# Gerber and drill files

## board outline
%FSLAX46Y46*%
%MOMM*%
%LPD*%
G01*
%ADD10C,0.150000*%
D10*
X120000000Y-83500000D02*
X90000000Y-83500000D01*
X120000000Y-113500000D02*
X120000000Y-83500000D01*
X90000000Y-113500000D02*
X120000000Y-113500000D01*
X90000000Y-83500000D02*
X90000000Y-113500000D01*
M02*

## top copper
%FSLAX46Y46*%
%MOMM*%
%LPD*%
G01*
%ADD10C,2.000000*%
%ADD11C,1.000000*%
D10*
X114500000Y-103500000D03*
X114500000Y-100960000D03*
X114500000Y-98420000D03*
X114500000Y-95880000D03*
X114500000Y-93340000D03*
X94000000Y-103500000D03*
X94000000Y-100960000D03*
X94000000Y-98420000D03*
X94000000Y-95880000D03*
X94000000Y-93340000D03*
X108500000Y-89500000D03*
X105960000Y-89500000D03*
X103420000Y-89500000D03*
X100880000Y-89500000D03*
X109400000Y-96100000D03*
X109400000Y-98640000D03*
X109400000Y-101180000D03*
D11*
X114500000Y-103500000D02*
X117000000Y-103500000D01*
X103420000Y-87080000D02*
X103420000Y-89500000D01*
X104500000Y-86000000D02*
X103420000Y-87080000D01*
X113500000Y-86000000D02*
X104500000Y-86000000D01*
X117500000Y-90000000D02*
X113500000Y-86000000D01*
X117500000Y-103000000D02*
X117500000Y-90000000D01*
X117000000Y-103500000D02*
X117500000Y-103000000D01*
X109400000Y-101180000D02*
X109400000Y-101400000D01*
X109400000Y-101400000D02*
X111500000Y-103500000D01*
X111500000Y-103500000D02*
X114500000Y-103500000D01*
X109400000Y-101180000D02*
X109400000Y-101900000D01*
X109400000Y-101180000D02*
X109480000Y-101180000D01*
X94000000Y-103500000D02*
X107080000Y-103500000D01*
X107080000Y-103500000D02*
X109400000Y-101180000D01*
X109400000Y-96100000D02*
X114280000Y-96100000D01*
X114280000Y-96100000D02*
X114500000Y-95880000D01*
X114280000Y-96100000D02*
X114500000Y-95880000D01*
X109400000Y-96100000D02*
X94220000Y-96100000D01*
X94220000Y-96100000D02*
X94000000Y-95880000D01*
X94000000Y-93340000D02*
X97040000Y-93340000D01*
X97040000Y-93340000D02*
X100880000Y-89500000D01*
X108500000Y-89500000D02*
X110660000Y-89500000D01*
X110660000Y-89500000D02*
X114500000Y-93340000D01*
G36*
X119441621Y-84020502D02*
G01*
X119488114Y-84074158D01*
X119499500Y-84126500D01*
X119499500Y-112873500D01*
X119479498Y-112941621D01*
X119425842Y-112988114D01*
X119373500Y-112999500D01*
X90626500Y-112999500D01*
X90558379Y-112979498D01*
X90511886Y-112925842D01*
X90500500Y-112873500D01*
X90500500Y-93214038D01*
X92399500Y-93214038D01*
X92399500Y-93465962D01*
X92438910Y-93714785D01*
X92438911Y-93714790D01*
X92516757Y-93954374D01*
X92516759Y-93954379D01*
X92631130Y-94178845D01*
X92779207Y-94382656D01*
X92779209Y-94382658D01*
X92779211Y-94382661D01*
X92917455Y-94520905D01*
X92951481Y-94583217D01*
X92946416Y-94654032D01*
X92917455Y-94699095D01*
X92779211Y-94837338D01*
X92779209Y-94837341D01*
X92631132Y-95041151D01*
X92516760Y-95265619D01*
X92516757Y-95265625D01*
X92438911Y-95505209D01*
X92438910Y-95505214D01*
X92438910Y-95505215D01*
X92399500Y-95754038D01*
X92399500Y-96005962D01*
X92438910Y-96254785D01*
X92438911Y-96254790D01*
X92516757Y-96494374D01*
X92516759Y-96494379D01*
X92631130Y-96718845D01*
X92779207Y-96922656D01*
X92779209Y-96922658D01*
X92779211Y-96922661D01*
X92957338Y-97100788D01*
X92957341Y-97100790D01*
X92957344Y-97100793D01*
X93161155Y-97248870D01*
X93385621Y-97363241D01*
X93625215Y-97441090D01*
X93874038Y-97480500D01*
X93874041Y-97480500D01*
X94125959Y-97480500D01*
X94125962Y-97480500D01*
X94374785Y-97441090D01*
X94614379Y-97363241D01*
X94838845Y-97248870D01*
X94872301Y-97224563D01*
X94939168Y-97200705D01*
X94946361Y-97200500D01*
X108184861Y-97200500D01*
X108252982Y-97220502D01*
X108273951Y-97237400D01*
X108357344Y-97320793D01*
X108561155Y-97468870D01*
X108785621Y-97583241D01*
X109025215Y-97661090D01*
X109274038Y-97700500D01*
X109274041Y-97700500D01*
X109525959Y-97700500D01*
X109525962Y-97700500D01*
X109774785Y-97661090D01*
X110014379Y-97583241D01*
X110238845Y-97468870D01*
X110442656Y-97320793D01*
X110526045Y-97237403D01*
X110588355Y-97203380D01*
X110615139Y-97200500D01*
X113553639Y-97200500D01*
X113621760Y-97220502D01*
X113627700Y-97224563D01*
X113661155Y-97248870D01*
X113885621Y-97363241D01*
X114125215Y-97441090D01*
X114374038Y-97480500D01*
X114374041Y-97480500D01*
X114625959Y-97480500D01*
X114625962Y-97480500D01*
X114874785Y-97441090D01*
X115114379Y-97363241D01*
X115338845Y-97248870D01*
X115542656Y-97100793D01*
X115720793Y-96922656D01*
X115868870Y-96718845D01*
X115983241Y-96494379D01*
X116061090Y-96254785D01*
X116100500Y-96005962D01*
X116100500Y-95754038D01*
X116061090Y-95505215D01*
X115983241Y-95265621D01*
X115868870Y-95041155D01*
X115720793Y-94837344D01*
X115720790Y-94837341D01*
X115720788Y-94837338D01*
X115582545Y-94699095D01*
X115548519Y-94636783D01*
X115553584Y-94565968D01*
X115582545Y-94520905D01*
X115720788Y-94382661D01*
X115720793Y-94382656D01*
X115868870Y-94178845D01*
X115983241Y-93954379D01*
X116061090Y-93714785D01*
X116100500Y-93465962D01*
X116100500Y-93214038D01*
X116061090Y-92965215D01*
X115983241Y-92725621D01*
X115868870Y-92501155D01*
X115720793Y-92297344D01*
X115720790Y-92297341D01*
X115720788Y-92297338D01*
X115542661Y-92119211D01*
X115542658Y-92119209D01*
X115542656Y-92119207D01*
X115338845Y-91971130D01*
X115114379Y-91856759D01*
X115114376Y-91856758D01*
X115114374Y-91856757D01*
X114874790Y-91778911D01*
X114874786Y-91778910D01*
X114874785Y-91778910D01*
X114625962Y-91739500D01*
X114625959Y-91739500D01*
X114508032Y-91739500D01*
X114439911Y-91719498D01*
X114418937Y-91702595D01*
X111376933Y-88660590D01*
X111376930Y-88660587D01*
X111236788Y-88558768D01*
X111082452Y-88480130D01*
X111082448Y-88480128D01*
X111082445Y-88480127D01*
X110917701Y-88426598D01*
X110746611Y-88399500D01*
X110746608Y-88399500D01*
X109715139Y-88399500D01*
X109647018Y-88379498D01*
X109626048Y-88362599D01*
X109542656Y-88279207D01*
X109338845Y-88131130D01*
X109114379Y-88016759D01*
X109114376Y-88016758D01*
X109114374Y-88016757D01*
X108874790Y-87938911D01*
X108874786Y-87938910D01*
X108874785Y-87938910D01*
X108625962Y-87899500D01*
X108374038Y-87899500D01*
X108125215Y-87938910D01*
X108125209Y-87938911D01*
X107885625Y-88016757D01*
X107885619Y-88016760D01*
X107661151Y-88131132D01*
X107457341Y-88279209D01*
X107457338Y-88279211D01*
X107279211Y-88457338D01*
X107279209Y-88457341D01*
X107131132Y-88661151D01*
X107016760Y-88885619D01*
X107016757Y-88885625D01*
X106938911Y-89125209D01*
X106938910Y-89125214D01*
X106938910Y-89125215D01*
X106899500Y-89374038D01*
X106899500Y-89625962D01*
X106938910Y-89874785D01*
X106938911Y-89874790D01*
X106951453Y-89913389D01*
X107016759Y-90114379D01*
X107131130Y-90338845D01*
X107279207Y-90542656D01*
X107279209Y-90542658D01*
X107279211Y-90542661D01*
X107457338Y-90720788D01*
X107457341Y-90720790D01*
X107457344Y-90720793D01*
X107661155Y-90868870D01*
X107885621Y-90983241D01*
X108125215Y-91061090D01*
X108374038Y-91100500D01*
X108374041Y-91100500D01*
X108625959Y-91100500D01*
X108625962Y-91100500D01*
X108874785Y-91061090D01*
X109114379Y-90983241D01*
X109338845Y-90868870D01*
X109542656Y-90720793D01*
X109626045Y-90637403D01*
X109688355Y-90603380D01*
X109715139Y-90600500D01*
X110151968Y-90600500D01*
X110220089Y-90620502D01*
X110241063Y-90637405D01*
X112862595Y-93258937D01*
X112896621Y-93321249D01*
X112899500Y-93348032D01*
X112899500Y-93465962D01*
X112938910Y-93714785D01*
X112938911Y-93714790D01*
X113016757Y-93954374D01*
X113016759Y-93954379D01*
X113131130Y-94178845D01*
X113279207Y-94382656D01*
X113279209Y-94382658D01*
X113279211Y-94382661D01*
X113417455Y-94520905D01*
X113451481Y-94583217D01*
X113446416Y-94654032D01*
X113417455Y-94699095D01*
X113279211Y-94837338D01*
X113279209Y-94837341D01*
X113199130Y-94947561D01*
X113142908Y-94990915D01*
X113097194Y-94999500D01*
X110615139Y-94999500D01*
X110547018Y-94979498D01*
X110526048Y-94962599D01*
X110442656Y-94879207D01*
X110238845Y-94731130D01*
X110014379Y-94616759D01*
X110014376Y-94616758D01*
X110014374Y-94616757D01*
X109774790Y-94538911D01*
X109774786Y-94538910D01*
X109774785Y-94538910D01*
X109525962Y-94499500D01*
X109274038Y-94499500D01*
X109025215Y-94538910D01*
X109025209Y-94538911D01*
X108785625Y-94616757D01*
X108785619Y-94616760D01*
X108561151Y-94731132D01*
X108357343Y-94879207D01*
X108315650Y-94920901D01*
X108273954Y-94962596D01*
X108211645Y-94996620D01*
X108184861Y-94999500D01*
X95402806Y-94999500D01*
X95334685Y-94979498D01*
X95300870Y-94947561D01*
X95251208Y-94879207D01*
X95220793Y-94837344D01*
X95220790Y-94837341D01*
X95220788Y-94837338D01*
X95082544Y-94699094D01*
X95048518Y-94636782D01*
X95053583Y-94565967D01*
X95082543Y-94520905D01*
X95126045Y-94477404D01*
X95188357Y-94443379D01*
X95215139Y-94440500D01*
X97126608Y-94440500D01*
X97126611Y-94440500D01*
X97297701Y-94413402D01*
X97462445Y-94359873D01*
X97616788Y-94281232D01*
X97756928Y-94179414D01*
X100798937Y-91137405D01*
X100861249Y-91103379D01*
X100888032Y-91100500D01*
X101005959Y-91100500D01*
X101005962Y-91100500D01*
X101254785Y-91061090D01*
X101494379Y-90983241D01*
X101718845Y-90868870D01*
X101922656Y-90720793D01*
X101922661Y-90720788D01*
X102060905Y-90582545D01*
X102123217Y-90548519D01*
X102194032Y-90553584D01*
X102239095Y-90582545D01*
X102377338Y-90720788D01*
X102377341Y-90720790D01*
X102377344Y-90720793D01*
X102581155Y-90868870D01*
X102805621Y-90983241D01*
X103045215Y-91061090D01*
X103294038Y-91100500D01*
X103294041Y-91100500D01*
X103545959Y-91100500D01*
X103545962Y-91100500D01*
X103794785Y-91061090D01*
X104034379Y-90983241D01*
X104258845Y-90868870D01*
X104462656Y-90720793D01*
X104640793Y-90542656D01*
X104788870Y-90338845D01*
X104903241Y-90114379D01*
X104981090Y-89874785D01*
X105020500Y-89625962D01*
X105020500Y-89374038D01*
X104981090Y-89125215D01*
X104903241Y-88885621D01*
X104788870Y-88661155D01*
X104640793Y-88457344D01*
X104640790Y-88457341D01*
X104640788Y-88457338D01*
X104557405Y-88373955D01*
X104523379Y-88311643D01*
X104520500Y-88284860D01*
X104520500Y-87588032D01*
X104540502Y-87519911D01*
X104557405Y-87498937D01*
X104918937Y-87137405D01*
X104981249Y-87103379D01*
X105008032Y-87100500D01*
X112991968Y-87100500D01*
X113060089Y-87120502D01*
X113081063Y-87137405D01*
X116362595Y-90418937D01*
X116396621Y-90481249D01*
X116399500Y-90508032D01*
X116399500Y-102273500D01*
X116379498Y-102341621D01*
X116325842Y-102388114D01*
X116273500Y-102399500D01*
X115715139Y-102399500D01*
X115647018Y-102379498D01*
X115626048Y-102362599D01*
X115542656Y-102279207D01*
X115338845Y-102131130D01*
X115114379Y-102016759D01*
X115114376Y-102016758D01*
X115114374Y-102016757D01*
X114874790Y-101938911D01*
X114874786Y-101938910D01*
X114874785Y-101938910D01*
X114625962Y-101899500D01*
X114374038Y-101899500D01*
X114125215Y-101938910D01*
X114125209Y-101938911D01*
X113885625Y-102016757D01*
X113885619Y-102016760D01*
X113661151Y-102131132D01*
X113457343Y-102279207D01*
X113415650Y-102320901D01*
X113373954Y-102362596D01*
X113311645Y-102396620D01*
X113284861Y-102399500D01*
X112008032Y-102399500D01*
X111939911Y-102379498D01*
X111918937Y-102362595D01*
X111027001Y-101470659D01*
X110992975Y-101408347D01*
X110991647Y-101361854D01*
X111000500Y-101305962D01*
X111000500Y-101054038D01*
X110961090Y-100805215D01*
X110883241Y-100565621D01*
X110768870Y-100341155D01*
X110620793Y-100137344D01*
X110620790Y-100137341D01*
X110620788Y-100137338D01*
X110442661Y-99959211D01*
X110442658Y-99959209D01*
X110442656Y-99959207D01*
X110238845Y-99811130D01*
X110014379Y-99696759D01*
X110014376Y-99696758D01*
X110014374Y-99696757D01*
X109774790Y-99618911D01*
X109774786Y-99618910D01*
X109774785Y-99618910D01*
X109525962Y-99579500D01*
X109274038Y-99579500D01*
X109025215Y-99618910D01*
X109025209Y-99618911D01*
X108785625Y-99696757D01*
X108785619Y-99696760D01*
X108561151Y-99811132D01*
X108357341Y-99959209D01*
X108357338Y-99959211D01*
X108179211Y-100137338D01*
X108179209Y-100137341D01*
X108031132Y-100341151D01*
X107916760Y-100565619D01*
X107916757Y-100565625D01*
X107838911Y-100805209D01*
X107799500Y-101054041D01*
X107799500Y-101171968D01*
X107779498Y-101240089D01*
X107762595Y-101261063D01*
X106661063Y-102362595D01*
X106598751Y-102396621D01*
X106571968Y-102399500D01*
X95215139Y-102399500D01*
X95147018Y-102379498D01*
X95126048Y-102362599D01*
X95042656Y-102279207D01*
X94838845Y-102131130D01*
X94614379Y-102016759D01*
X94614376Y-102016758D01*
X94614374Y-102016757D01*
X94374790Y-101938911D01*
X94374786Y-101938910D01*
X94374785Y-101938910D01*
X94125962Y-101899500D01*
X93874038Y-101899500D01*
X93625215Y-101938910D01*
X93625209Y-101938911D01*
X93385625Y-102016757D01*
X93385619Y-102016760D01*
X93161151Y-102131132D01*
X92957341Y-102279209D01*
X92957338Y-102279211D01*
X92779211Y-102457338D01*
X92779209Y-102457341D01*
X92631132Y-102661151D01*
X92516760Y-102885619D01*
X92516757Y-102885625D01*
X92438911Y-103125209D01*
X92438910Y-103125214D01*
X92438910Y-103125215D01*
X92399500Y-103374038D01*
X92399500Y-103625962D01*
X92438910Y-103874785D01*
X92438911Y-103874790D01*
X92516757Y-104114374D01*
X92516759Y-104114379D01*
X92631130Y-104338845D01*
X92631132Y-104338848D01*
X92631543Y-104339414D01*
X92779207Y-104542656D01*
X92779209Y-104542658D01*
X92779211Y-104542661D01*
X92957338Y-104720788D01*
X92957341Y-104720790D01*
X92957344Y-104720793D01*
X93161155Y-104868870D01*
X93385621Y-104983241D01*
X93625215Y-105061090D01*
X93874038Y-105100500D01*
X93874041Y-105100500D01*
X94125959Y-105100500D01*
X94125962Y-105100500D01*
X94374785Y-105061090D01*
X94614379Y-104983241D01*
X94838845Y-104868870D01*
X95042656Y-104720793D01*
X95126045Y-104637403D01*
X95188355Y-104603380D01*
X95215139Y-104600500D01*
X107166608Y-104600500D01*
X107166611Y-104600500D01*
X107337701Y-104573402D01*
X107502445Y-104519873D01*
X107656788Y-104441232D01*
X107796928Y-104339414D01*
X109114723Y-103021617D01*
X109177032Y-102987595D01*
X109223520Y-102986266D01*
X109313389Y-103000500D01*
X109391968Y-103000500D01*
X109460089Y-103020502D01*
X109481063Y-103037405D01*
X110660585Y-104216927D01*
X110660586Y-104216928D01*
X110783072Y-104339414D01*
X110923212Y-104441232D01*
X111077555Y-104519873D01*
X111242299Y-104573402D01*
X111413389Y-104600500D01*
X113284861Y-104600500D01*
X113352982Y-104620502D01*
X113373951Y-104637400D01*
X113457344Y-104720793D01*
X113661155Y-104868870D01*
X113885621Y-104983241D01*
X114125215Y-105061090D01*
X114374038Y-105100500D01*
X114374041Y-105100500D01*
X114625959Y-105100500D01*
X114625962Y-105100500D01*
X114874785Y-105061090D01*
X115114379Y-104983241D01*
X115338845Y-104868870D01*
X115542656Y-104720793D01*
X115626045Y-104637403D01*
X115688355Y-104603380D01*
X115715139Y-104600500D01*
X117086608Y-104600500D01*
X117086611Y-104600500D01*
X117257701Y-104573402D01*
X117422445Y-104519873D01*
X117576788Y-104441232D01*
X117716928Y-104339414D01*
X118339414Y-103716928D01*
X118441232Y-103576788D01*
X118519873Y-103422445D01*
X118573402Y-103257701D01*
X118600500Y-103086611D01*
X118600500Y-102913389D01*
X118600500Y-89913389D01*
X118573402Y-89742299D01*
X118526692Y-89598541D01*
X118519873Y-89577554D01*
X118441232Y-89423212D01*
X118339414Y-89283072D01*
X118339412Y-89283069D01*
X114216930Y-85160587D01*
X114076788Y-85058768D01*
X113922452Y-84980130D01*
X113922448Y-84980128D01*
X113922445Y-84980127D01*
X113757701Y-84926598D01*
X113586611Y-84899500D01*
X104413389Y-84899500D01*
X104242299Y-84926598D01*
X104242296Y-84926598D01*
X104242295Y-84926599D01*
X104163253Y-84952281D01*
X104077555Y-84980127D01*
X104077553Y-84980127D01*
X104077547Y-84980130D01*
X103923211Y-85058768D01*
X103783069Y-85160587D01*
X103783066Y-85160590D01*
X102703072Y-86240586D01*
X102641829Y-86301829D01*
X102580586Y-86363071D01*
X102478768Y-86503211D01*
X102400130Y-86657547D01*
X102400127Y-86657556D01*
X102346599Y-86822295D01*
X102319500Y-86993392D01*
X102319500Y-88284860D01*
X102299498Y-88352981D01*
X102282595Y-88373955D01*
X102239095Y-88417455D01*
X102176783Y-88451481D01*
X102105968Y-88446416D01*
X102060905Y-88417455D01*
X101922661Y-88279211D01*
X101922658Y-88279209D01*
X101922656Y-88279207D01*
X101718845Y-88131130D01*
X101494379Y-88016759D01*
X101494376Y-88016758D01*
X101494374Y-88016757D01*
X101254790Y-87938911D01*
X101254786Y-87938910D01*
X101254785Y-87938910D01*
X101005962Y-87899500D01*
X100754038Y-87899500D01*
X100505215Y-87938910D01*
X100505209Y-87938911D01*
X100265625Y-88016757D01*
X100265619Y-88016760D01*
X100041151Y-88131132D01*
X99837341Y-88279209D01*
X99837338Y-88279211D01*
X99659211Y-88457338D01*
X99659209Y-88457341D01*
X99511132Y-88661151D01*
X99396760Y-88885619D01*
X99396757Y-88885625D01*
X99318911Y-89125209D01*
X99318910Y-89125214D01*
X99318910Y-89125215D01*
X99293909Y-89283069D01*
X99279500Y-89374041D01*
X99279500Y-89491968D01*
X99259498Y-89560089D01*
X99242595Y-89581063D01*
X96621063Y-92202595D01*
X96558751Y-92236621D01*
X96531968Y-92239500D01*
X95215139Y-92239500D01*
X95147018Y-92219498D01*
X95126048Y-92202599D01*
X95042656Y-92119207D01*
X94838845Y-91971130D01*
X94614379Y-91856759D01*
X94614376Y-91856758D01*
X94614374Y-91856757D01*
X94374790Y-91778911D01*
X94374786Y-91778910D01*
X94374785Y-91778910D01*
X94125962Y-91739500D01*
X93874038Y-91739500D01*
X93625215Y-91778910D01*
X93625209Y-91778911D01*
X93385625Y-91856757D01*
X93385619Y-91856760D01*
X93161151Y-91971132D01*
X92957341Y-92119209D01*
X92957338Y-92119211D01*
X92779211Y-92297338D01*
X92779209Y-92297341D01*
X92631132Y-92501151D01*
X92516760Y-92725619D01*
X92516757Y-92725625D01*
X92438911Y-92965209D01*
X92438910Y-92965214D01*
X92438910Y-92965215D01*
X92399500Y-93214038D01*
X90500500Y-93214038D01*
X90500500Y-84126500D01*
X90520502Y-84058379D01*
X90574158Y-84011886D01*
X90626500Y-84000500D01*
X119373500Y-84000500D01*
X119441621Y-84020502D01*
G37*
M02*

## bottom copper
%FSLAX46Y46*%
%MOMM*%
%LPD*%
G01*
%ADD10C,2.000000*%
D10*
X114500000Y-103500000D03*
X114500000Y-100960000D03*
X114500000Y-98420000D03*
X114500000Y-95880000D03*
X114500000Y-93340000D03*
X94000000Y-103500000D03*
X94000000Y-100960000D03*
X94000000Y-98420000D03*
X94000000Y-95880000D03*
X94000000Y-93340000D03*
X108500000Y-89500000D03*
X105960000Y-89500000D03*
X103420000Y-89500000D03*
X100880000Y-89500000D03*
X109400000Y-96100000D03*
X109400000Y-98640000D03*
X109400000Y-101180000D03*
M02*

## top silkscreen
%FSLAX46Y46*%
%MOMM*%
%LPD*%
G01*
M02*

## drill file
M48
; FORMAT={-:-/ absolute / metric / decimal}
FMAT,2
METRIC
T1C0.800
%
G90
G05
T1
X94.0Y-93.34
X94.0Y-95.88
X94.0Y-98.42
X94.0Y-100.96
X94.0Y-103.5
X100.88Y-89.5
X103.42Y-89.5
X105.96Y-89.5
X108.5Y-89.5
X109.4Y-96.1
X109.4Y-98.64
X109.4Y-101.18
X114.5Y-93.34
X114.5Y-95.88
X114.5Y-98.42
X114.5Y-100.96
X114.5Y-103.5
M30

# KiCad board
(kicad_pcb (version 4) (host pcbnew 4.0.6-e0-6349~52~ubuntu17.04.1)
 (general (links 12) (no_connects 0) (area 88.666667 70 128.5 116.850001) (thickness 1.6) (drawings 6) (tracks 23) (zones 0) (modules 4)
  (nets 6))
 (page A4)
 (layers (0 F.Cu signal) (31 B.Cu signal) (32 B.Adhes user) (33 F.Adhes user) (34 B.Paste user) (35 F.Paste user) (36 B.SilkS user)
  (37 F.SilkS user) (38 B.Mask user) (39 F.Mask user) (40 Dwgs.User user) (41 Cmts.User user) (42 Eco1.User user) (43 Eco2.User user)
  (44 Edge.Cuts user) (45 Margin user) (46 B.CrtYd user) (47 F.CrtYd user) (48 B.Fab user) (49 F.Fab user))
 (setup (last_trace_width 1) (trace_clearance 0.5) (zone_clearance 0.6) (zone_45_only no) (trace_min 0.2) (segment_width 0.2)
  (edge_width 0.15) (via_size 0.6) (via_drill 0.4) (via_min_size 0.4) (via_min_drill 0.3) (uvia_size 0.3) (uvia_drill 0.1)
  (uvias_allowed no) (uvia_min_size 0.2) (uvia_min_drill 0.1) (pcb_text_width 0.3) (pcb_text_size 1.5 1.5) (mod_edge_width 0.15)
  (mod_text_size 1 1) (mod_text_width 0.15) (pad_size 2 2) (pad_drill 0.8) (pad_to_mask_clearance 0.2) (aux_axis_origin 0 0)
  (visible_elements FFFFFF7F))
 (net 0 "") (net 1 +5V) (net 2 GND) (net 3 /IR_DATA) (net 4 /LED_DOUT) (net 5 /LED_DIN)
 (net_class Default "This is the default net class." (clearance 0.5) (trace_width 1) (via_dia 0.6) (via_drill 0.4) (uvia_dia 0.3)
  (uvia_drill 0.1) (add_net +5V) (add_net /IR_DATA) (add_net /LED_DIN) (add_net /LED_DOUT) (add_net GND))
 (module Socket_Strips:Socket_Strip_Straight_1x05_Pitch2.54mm (layer B.Cu) (at 114.5 103.5)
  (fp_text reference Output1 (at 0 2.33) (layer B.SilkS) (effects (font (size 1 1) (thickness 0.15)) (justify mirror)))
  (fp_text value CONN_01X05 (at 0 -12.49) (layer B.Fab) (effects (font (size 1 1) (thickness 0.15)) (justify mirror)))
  (pad 1 thru_hole circle (at 0 0) (size 2 2) (drill 0.8) (layers *.Cu *.Mask) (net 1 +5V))
  (pad 2 thru_hole circle (at 0 -2.54) (size 2 2) (drill 0.8) (layers *.Cu *.Mask) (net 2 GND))
  (pad 3 thru_hole circle (at 0 -5.08) (size 2 2) (drill 0.8) (layers *.Cu *.Mask) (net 2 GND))
  (pad 4 thru_hole circle (at 0 -7.62) (size 2 2) (drill 0.8) (layers *.Cu *.Mask) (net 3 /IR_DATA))
  (pad 5 thru_hole circle (at 0 -10.16) (size 2 2) (drill 0.8) (layers *.Cu *.Mask) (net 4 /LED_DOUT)))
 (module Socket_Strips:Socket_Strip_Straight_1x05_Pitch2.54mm (layer B.Cu) (at 94 103.5)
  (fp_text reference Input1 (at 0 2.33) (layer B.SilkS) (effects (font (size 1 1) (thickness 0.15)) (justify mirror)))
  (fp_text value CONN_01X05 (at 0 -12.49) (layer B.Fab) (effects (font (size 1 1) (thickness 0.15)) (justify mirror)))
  (pad 1 thru_hole circle (at 0 0) (size 2 2) (drill 0.8) (layers *.Cu *.Mask) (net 1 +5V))
  (pad 2 thru_hole circle (at 0 -2.54) (size 2 2) (drill 0.8) (layers *.Cu *.Mask) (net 2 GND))
  (pad 3 thru_hole circle (at 0 -5.08) (size 2 2) (drill 0.8) (layers *.Cu *.Mask) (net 2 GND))
  (pad 4 thru_hole circle (at 0 -7.62) (size 2 2) (drill 0.8) (layers *.Cu *.Mask) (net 3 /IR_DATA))
  (pad 5 thru_hole circle (at 0 -10.16) (size 2 2) (drill 0.8) (layers *.Cu *.Mask) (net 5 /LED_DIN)))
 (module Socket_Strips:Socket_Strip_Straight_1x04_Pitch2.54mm (layer B.Cu) (at 108.5 89.5 90)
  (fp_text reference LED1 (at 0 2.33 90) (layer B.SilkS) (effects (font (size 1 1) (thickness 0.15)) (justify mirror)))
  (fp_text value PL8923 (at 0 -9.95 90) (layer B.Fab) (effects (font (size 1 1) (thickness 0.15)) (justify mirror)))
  (pad 1 thru_hole circle (at 0 0 90) (size 2 2) (drill 0.8) (layers *.Cu *.Mask) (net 4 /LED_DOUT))
  (pad 2 thru_hole circle (at 0 -2.54 90) (size 2 2) (drill 0.8) (layers *.Cu *.Mask) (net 2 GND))
  (pad 3 thru_hole circle (at 0 -5.08 90) (size 2 2) (drill 0.8) (layers *.Cu *.Mask) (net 1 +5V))
  (pad 4 thru_hole circle (at 0 -7.62 90) (size 2 2) (drill 0.8) (layers *.Cu *.Mask) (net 5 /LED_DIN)))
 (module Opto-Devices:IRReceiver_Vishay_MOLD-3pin (layer B.Cu) (at 109.4 96.1 270)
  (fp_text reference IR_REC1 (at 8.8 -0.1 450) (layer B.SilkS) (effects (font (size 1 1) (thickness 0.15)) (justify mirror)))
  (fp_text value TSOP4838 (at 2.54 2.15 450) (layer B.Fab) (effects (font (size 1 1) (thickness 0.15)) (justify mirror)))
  (pad 1 thru_hole circle (at 0 0 270) (size 2 2) (drill 0.8) (layers *.Cu *.Mask) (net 3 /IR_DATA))
  (pad 2 thru_hole circle (at 2.54 0 270) (size 2 2) (drill 0.8) (layers *.Cu *.Mask) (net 2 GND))
  (pad 3 thru_hole circle (at 5.08 0 270) (size 2 2) (drill 0.8) (layers *.Cu *.Mask) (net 1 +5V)))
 (gr_line (start 120 83.5) (end 90 83.5) (angle 90) (layer Edge.Cuts) (width 0.15))
 (gr_line (start 120 113.5) (end 120 83.5) (angle 90) (layer Edge.Cuts) (width 0.15))
 (gr_line (start 90 113.5) (end 120 113.5) (angle 90) (layer Edge.Cuts) (width 0.15))
 (gr_line (start 90 83.5) (end 90 113.5) (angle 90) (layer Edge.Cuts) (width 0.15))
 (segment (start 114.5 103.5) (end 117 103.5) (width 1) (layer F.Cu) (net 1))
 (segment (start 103.42 87.08) (end 103.42 89.5) (width 1) (layer F.Cu) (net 1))
 (segment (start 104.5 86) (end 103.42 87.08) (width 1) (layer F.Cu) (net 1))
 (segment (start 113.5 86) (end 104.5 86) (width 1) (layer F.Cu) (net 1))
 (segment (start 117.5 90) (end 113.5 86) (width 1) (layer F.Cu) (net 1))
 (segment (start 117.5 103) (end 117.5 90) (width 1) (layer F.Cu) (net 1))
 (segment (start 117 103.5) (end 117.5 103) (width 1) (layer F.Cu) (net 1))
 (segment (start 109.4 101.18) (end 109.4 101.4) (width 1) (layer F.Cu) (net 1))
 (segment (start 109.4 101.4) (end 111.5 103.5) (width 1) (layer F.Cu) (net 1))
 (segment (start 111.5 103.5) (end 114.5 103.5) (width 1) (layer F.Cu) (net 1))
 (segment (start 109.4 101.18) (end 109.4 101.9) (width 1) (layer F.Cu) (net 1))
 (segment (start 109.4 101.18) (end 109.48 101.18) (width 1) (layer F.Cu) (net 1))
 (segment (start 94 103.5) (end 107.08 103.5) (width 1) (layer F.Cu) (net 1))
 (segment (start 107.08 103.5) (end 109.4 101.18) (width 1) (layer F.Cu) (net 1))
 (segment (start 109.4 96.1) (end 114.28 96.1) (width 1) (layer F.Cu) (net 3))
 (segment (start 114.28 96.1) (end 114.5 95.88) (width 1) (layer F.Cu) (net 3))
 (segment (start 114.28 96.1) (end 114.5 95.88) (width 1) (layer F.Cu) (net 3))
 (segment (start 109.4 96.1) (end 94.22 96.1) (width 1) (layer F.Cu) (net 3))
 (segment (start 94.22 96.1) (end 94 95.88) (width 1) (layer F.Cu) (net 3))
 (segment (start 94 93.34) (end 97.04 93.34) (width 1) (layer F.Cu) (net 5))
 (segment (start 97.04 93.34) (end 100.88 89.5) (width 1) (layer F.Cu) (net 5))
 (segment (start 108.5 89.5) (end 110.66 89.5) (width 1) (layer F.Cu) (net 4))
 (segment (start 110.66 89.5) (end 114.5 93.34) (width 1) (layer F.Cu) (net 4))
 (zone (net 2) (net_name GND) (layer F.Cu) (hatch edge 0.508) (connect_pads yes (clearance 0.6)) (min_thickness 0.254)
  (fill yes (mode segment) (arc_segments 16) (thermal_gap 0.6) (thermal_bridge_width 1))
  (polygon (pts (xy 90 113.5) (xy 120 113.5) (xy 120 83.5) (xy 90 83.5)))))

